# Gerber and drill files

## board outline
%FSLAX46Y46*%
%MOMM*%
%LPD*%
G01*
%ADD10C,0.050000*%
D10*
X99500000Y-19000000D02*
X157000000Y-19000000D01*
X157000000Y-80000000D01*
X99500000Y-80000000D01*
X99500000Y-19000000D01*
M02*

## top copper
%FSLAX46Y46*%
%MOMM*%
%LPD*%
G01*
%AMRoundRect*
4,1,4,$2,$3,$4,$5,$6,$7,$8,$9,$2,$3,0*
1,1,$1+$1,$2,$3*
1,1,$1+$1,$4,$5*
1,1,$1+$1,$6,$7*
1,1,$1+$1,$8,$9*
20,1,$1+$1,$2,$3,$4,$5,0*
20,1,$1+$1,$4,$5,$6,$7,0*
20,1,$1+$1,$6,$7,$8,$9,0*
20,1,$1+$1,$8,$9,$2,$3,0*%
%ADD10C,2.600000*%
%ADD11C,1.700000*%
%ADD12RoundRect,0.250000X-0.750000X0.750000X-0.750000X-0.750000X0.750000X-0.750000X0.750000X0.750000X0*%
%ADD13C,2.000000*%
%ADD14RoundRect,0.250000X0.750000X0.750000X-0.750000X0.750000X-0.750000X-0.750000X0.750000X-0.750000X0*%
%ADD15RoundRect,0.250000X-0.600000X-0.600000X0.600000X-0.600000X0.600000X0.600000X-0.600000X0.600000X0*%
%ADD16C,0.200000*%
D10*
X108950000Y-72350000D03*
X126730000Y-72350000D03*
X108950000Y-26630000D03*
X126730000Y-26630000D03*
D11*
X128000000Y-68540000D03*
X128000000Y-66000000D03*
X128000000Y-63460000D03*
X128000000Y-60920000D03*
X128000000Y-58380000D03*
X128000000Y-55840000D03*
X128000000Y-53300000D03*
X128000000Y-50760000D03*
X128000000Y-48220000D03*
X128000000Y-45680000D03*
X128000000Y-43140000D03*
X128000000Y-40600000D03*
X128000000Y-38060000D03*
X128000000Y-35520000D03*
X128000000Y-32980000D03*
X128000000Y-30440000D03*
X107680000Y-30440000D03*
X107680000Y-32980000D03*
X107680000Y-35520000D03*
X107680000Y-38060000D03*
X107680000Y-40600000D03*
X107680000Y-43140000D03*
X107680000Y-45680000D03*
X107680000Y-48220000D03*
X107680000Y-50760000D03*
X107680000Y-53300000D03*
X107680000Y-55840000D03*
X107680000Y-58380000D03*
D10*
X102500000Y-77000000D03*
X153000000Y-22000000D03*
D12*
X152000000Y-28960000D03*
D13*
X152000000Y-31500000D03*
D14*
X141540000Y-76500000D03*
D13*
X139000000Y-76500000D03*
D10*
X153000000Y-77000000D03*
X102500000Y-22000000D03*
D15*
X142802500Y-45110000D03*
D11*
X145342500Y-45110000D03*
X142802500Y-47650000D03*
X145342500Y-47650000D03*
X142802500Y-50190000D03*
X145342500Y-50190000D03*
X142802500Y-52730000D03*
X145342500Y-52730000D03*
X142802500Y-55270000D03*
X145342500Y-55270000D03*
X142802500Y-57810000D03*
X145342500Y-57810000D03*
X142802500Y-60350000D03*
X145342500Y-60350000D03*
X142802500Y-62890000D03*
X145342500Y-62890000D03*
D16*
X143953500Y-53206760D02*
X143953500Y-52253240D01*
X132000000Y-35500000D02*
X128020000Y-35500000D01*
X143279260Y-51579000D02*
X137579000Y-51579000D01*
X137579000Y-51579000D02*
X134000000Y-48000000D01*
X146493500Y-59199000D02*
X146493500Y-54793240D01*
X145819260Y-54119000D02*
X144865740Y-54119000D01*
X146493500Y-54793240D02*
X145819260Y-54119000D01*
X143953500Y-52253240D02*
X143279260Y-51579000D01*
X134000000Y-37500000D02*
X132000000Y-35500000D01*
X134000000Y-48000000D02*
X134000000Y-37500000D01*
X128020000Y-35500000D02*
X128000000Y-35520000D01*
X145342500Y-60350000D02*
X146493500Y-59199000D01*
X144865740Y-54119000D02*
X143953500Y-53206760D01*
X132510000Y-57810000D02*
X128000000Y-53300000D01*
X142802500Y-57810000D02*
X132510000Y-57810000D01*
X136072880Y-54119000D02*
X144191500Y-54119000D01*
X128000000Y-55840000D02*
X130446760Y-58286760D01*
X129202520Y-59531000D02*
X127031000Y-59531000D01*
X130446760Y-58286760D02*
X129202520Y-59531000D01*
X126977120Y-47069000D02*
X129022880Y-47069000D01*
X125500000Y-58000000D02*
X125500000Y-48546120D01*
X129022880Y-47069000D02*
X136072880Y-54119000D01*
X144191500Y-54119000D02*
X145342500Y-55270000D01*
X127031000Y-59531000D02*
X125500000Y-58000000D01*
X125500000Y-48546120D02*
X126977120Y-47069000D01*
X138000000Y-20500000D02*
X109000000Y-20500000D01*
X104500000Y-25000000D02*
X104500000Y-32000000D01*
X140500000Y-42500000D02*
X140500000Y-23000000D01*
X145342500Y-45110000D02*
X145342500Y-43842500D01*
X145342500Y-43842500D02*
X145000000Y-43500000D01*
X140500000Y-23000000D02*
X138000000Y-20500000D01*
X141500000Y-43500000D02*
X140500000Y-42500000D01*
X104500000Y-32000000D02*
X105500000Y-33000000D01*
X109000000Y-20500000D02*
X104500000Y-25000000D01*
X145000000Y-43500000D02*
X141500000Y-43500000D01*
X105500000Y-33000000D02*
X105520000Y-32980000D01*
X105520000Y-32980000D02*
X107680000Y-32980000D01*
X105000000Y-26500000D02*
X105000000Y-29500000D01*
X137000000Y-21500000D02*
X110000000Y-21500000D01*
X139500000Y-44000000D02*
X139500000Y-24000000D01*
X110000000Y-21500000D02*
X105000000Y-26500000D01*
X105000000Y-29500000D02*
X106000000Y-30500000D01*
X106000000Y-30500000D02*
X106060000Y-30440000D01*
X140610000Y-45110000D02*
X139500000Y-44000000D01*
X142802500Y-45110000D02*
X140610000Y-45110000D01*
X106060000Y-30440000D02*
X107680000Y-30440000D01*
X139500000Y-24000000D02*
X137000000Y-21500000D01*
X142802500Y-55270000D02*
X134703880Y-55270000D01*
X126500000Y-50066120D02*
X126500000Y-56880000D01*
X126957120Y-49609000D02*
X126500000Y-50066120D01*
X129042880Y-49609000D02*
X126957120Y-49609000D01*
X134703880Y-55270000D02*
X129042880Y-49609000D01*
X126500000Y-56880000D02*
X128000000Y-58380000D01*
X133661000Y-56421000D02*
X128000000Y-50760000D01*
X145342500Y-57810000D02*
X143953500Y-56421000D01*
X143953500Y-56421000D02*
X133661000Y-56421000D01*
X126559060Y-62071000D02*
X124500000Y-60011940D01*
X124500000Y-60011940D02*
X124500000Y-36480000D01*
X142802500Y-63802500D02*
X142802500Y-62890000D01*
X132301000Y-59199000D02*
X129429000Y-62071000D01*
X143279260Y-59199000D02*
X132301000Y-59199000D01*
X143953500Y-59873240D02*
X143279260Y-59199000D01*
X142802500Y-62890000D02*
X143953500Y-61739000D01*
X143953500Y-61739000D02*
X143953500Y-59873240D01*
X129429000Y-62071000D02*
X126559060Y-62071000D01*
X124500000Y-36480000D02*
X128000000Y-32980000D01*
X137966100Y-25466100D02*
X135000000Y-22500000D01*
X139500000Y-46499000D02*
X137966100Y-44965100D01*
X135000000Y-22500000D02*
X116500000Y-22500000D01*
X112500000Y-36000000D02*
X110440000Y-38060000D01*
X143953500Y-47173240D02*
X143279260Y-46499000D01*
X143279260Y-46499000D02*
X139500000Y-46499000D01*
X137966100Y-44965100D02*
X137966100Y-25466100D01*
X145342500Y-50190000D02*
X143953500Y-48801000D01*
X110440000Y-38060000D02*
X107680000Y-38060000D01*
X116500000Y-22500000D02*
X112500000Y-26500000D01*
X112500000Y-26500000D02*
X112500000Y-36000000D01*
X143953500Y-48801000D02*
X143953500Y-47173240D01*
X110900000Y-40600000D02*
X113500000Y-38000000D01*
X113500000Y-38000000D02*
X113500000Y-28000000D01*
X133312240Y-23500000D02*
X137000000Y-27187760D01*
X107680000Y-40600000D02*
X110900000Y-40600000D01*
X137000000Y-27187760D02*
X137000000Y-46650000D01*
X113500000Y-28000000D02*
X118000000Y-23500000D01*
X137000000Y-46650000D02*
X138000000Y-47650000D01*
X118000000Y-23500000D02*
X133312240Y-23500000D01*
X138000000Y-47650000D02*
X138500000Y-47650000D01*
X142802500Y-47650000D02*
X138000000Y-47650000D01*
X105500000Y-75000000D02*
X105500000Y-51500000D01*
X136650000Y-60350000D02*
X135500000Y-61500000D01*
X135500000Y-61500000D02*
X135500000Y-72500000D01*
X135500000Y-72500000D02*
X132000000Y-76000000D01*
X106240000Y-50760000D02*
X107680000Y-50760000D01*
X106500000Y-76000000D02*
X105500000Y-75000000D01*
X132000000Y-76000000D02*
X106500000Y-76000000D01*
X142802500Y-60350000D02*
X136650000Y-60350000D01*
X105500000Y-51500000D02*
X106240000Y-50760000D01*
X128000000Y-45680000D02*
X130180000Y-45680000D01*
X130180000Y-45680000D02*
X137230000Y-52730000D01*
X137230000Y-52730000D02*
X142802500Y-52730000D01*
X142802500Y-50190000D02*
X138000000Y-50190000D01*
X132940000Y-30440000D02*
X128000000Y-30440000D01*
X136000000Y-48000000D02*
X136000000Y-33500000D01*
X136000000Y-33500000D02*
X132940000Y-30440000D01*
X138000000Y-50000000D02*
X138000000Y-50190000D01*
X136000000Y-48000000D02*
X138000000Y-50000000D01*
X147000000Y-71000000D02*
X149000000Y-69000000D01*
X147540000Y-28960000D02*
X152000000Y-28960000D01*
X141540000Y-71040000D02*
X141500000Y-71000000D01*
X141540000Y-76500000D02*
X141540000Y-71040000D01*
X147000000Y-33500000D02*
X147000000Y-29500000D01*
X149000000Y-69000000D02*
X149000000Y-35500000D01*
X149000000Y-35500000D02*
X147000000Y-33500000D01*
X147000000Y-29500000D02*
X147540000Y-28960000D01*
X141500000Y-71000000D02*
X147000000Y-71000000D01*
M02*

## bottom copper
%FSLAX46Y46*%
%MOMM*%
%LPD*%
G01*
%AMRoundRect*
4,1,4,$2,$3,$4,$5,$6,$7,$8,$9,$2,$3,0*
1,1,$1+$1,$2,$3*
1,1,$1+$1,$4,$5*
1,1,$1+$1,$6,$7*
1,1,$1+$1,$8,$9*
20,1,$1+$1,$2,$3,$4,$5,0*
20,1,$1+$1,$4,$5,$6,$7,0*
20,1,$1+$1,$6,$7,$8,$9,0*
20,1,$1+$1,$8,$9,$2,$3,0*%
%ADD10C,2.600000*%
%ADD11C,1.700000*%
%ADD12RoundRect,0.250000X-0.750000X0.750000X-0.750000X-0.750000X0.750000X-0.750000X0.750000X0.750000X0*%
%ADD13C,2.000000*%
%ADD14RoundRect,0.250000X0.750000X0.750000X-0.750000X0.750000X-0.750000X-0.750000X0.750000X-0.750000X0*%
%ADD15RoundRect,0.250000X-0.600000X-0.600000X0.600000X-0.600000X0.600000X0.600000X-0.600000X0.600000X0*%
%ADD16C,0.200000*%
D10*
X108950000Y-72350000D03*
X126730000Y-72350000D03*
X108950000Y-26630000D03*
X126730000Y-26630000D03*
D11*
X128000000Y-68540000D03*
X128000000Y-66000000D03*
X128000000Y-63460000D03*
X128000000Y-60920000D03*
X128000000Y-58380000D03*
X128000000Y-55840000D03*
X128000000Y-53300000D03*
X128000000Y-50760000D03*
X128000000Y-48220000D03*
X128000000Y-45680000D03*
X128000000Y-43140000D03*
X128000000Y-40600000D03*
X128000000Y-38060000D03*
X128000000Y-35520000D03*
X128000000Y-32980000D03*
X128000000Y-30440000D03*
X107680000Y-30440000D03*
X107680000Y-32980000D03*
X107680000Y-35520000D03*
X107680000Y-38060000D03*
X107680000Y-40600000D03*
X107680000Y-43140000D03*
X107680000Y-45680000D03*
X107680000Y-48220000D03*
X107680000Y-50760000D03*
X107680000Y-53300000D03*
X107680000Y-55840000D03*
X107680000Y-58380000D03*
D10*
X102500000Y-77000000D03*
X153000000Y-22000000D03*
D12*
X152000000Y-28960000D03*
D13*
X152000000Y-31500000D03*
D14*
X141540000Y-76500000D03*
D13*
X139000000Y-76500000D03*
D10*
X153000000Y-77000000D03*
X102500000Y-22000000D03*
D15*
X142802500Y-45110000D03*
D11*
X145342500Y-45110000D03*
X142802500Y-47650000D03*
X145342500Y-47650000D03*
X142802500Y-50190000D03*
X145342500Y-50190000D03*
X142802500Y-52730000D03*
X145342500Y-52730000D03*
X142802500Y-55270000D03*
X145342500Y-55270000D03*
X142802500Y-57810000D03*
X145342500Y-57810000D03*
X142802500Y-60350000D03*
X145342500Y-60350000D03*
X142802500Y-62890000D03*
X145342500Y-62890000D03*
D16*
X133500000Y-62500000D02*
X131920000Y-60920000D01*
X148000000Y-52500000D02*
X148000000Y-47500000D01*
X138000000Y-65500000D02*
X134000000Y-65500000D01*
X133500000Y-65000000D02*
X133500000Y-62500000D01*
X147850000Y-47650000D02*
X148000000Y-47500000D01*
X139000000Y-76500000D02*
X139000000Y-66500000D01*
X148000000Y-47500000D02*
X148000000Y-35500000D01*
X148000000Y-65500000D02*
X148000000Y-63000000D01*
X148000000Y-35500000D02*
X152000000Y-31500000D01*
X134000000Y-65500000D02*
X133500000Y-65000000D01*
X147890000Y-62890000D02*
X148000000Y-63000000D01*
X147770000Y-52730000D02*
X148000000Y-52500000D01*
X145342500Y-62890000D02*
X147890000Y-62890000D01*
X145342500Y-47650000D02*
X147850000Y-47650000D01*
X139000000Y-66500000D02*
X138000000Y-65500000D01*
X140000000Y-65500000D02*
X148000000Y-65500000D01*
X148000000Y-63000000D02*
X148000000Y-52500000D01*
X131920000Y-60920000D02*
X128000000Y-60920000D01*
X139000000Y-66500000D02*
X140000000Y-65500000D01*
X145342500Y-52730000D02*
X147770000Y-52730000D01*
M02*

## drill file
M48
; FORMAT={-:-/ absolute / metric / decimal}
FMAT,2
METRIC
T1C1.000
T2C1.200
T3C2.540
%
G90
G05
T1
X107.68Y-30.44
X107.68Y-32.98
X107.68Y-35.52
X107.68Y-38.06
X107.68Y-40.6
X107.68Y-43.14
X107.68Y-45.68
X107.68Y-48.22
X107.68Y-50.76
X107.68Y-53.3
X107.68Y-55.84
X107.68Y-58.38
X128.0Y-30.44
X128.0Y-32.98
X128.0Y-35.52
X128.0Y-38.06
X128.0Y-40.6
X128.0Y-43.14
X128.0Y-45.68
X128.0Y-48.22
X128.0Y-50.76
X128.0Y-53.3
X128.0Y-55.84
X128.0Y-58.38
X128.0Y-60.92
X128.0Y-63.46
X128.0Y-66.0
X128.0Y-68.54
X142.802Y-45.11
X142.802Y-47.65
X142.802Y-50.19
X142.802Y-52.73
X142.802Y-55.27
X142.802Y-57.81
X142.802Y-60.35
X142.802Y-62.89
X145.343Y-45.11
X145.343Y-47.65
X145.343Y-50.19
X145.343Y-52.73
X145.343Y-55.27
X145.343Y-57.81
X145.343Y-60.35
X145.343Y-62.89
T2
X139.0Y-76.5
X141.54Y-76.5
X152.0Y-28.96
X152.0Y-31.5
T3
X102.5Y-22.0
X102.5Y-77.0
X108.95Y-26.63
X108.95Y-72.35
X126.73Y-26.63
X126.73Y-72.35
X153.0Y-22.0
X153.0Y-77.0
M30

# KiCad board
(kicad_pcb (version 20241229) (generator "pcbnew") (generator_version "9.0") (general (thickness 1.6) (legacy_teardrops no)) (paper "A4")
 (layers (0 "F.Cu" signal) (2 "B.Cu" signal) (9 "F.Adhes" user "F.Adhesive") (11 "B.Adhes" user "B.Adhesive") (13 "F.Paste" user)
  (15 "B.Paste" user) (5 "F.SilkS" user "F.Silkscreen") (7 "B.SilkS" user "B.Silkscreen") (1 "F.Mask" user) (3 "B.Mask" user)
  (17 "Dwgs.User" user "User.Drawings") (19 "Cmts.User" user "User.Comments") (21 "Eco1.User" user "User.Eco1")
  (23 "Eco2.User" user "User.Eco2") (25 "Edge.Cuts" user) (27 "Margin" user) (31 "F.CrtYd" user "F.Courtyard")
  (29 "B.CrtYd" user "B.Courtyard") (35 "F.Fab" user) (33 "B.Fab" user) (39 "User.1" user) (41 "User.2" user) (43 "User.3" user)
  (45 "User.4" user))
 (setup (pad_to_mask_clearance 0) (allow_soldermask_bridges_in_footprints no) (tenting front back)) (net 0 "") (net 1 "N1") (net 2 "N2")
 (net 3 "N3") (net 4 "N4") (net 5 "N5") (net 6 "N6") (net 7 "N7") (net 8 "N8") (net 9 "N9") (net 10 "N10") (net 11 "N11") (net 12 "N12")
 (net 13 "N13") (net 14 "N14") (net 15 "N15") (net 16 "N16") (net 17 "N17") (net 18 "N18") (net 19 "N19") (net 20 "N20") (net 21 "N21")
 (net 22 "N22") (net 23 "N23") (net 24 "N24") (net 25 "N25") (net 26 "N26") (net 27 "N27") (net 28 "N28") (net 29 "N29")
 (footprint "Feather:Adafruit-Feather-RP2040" (layer "F.Cu") (at 117.84 49.49 90)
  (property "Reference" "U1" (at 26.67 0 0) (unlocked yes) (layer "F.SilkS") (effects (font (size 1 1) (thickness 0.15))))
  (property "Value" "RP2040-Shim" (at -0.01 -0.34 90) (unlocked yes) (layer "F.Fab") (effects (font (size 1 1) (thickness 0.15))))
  (pad "" np_thru_hole circle (at -22.86 -8.89 90) (size 2.6 2.6) (drill 2.54) (layers "*.Cu" "*.Mask") (solder_mask_margin 1.3)
   (clearance 1.3))
  (pad "" np_thru_hole circle (at -22.86 8.89 90) (size 2.6 2.6) (drill 2.54) (layers "*.Cu" "*.Mask") (solder_mask_margin 1.3)
   (clearance 1.3))
  (pad "" np_thru_hole circle (at 22.86 -8.89 90) (size 2.6 2.6) (drill 2.54) (layers "*.Cu" "*.Mask") (solder_mask_margin 1.3)
   (clearance 1.3))
  (pad "" np_thru_hole circle (at 22.86 8.89 90) (size 2.6 2.6) (drill 2.54) (layers "*.Cu" "*.Mask") (solder_mask_margin 1.3)
   (clearance 1.3))
  (pad "1" thru_hole circle (at -19.05 10.16 90) (size 1.7 1.7) (drill 1) (layers "*.Cu" "*.Mask") (remove_unused_layers no) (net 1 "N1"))
  (pad "2" thru_hole circle (at -16.51 10.16 90) (size 1.7 1.7) (drill 1) (layers "*.Cu" "*.Mask") (remove_unused_layers no) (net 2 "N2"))
  (pad "3" thru_hole circle (at -13.97 10.16 90) (size 1.7 1.7) (drill 1) (layers "*.Cu" "*.Mask") (remove_unused_layers no) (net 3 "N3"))
  (pad "4" thru_hole circle (at -11.43 10.16 90) (size 1.7 1.7) (drill 1) (layers "*.Cu" "*.Mask") (remove_unused_layers no) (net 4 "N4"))
  (pad "5" thru_hole circle (at -8.89 10.16 90) (size 1.7 1.7) (drill 1) (layers "*.Cu" "*.Mask") (remove_unused_layers no) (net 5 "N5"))
  (pad "6" thru_hole circle (at -6.35 10.16 90) (size 1.7 1.7) (drill 1) (layers "*.Cu" "*.Mask") (remove_unused_layers no) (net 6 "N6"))
  (pad "7" thru_hole circle (at -3.81 10.16 90) (size 1.7 1.7) (drill 1) (layers "*.Cu" "*.Mask") (remove_unused_layers no) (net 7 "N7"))
  (pad "8" thru_hole circle (at -1.27 10.16 90) (size 1.7 1.7) (drill 1) (layers "*.Cu" "*.Mask") (remove_unused_layers no) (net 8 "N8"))
  (pad "9" thru_hole circle (at 1.27 10.16 90) (size 1.7 1.7) (drill 1) (layers "*.Cu" "*.Mask") (remove_unused_layers no) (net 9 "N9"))
  (pad "10" thru_hole circle (at 3.81 10.16 90) (size 1.7 1.7) (drill 1) (layers "*.Cu" "*.Mask") (remove_unused_layers no) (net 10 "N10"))
  (pad "11" thru_hole circle (at 6.35 10.16 90) (size 1.7 1.7) (drill 1) (layers "*.Cu" "*.Mask") (remove_unused_layers no) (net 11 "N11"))
  (pad "12" thru_hole circle (at 8.89 10.16 90) (size 1.7 1.7) (drill 1) (layers "*.Cu" "*.Mask") (remove_unused_layers no) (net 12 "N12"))
  (pad "13" thru_hole circle (at 11.43 10.16 90) (size 1.7 1.7) (drill 1) (layers "*.Cu" "*.Mask") (remove_unused_layers no) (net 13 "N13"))
  (pad "14" thru_hole circle (at 13.97 10.16 90) (size 1.7 1.7) (drill 1) (layers "*.Cu" "*.Mask") (remove_unused_layers no) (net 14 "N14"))
  (pad "15" thru_hole circle (at 16.51 10.16 90) (size 1.7 1.7) (drill 1) (layers "*.Cu" "*.Mask") (remove_unused_layers no) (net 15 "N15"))
  (pad "16" thru_hole circle (at 19.05 10.16 90) (size 1.7 1.7) (drill 1) (layers "*.Cu" "*.Mask") (remove_unused_layers no) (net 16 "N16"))
  (pad "17" thru_hole circle (at 19.05 -10.16 90) (size 1.7 1.7) (drill 1) (layers "*.Cu" "*.Mask") (remove_unused_layers no) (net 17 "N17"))
  (pad "18" thru_hole circle (at 16.51 -10.16 90) (size 1.7 1.7) (drill 1) (layers "*.Cu" "*.Mask") (remove_unused_layers no) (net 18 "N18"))
  (pad "19" thru_hole circle (at 13.97 -10.16 90) (size 1.7 1.7) (drill 1) (layers "*.Cu" "*.Mask") (remove_unused_layers no) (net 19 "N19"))
  (pad "20" thru_hole circle (at 11.43 -10.16 90) (size 1.7 1.7) (drill 1) (layers "*.Cu" "*.Mask") (remove_unused_layers no) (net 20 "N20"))
  (pad "21" thru_hole circle (at 8.89 -10.16 90) (size 1.7 1.7) (drill 1) (layers "*.Cu" "*.Mask") (remove_unused_layers no) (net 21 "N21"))
  (pad "22" thru_hole circle (at 6.35 -10.16 90) (size 1.7 1.7) (drill 1) (layers "*.Cu" "*.Mask") (remove_unused_layers no) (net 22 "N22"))
  (pad "23" thru_hole circle (at 3.81 -10.16 90) (size 1.7 1.7) (drill 1) (layers "*.Cu" "*.Mask") (remove_unused_layers no) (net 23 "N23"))
  (pad "24" thru_hole circle (at 1.27 -10.16 90) (size 1.7 1.7) (drill 1) (layers "*.Cu" "*.Mask") (remove_unused_layers no) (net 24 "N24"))
  (pad "25" thru_hole circle (at -1.27 -10.16 90) (size 1.7 1.7) (drill 1) (layers "*.Cu" "*.Mask") (remove_unused_layers no) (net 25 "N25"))
  (pad "26" thru_hole circle (at -3.81 -10.16 90) (size 1.7 1.7) (drill 1) (layers "*.Cu" "*.Mask") (remove_unused_layers no) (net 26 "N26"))
  (pad "27" thru_hole circle (at -6.35 -10.16 90) (size 1.7 1.7) (drill 1) (layers "*.Cu" "*.Mask") (remove_unused_layers no) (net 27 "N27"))
  (pad "28" thru_hole circle (at -8.89 -10.16 90) (size 1.7 1.7) (drill 1) (layers "*.Cu" "*.Mask") (remove_unused_layers no) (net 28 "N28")))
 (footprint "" (layer "F.Cu") (at 102.5 77)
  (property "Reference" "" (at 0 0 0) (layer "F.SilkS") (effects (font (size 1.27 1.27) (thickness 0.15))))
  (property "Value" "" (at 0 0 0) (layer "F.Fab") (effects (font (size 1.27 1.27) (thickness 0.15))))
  (pad "" np_thru_hole circle (at 0 0 90) (size 2.6 2.6) (drill 2.54) (layers "*.Cu" "*.Mask") (solder_mask_margin 1.3) (clearance 1.3)))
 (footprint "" (layer "F.Cu") (at 153 22)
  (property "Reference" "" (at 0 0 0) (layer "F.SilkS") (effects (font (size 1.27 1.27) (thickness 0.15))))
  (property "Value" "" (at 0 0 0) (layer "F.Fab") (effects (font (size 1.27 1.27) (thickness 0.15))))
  (pad "" np_thru_hole circle (at 0 0 90) (size 2.6 2.6) (drill 2.54) (layers "*.Cu" "*.Mask") (solder_mask_margin 1.3) (clearance 1.3)))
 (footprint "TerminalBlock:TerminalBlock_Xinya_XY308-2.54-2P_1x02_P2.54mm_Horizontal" (layer "F.Cu") (at 152 28.96 -90)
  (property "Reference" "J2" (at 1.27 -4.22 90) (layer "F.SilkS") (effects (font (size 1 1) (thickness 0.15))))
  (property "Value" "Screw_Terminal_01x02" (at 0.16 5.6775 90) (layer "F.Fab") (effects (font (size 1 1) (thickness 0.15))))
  (pad "1" thru_hole roundrect (at 0 0 270) (size 2 2) (drill 1.2) (layers "*.Cu" "*.Mask") (remove_unused_layers no)
   (roundrect_rratio 0.125) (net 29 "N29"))
  (pad "2" thru_hole circle (at 2.54 0 270) (size 2 2) (drill 1.2) (layers "*.Cu" "*.Mask") (remove_unused_layers no) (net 4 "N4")))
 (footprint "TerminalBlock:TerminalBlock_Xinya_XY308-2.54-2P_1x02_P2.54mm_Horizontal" (layer "F.Cu") (at 141.54 76.5 180)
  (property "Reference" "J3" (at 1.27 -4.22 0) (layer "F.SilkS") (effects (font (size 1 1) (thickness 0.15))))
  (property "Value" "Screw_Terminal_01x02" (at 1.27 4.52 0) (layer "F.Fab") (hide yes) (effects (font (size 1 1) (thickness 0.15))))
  (pad "1" thru_hole roundrect (at 0 0 180) (size 2 2) (drill 1.2) (layers "*.Cu" "*.Mask") (remove_unused_layers no)
   (roundrect_rratio 0.125) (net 29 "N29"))
  (pad "2" thru_hole circle (at 2.54 0 180) (size 2 2) (drill 1.2) (layers "*.Cu" "*.Mask") (remove_unused_layers no) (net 4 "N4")))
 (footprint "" (layer "F.Cu") (at 153 77)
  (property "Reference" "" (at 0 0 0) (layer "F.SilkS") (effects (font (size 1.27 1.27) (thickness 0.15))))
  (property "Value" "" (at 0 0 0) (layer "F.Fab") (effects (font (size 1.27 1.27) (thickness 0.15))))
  (pad "" np_thru_hole circle (at 0 0 90) (size 2.6 2.6) (drill 2.54) (layers "*.Cu" "*.Mask") (solder_mask_margin 1.3) (clearance 1.3)))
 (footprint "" (layer "F.Cu") (at 102.5 22)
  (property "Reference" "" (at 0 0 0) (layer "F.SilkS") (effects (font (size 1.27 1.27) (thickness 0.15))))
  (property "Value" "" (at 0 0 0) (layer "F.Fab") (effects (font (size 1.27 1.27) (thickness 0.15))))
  (pad "" np_thru_hole circle (at 0 0 90) (size 2.6 2.6) (drill 2.54) (layers "*.Cu" "*.Mask") (solder_mask_margin 1.3) (clearance 1.3)))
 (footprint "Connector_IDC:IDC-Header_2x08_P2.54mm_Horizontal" (layer "F.Cu") (at 142.8025 45.11)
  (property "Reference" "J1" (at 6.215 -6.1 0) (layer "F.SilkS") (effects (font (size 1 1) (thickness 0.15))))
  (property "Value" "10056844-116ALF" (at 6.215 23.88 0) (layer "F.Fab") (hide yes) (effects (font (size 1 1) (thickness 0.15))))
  (pad "1" thru_hole roundrect (at 0 0) (size 1.7 1.7) (drill 1) (layers "*.Cu" "*.Mask") (remove_unused_layers no)
   (roundrect_rratio 0.147059) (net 17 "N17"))
  (pad "2" thru_hole circle (at 2.54 0) (size 1.7 1.7) (drill 1) (layers "*.Cu" "*.Mask") (remove_unused_layers no) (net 18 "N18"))
  (pad "3" thru_hole circle (at 0 2.54) (size 1.7 1.7) (drill 1) (layers "*.Cu" "*.Mask") (remove_unused_layers no) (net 21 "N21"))
  (pad "4" thru_hole circle (at 2.54 2.54) (size 1.7 1.7) (drill 1) (layers "*.Cu" "*.Mask") (remove_unused_layers no) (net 4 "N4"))
  (pad "5" thru_hole circle (at 0 5.08) (size 1.7 1.7) (drill 1) (layers "*.Cu" "*.Mask") (remove_unused_layers no) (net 16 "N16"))
  (pad "6" thru_hole circle (at 2.54 5.08) (size 1.7 1.7) (drill 1) (layers "*.Cu" "*.Mask") (remove_unused_layers no) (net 20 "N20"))
  (pad "7" thru_hole circle (at 0 7.62) (size 1.7 1.7) (drill 1) (layers "*.Cu" "*.Mask") (remove_unused_layers no) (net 10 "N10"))
  (pad "8" thru_hole circle (at 2.54 7.62) (size 1.7 1.7) (drill 1) (layers "*.Cu" "*.Mask") (remove_unused_layers no) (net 4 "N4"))
  (pad "9" thru_hole circle (at 0 10.16) (size 1.7 1.7) (drill 1) (layers "*.Cu" "*.Mask") (remove_unused_layers no) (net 5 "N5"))
  (pad "10" thru_hole circle (at 2.54 10.16) (size 1.7 1.7) (drill 1) (layers "*.Cu" "*.Mask") (remove_unused_layers no) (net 6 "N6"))
  (pad "11" thru_hole circle (at 0 12.7) (size 1.7 1.7) (drill 1) (layers "*.Cu" "*.Mask") (remove_unused_layers no) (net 7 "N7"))
  (pad "12" thru_hole circle (at 2.54 12.7) (size 1.7 1.7) (drill 1) (layers "*.Cu" "*.Mask") (remove_unused_layers no) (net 8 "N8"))
  (pad "13" thru_hole circle (at 0 15.24) (size 1.7 1.7) (drill 1) (layers "*.Cu" "*.Mask") (remove_unused_layers no) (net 25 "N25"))
  (pad "14" thru_hole circle (at 2.54 15.24) (size 1.7 1.7) (drill 1) (layers "*.Cu" "*.Mask") (remove_unused_layers no) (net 14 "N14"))
  (pad "15" thru_hole circle (at 0 17.78) (size 1.7 1.7) (drill 1) (layers "*.Cu" "*.Mask") (remove_unused_layers no) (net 15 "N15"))
  (pad "16" thru_hole circle (at 2.54 17.78) (size 1.7 1.7) (drill 1) (layers "*.Cu" "*.Mask") (remove_unused_layers no) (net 4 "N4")))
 (gr_rect (start 99.5 19) (end 157 80) (stroke (width 0.05) (type solid)) (fill no) (layer "Edge.Cuts"))
 (segment (start 143.9535 53.20676) (end 143.9535 52.25324) (width 0.2) (layer "F.Cu") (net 14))
 (segment (start 132 35.5) (end 128.02 35.5) (width 0.2) (layer "F.Cu") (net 14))
 (segment (start 143.27926 51.579) (end 137.579 51.579) (width 0.2) (layer "F.Cu") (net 14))
 (segment (start 137.579 51.579) (end 134 48) (width 0.2) (layer "F.Cu") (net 14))
 (segment (start 146.4935 59.199) (end 146.4935 54.79324) (width 0.2) (layer "F.Cu") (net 14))
 (segment (start 145.81926 54.119) (end 144.86574 54.119) (width 0.2) (layer "F.Cu") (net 14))
 (segment (start 146.4935 54.79324) (end 145.81926 54.119) (width 0.2) (layer "F.Cu") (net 14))
 (segment (start 143.9535 52.25324) (end 143.27926 51.579) (width 0.2) (layer "F.Cu") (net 14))
 (segment (start 134 37.5) (end 132 35.5) (width 0.2) (layer "F.Cu") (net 14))
 (segment (start 134 48) (end 134 37.5) (width 0.2) (layer "F.Cu") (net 14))
 (segment (start 128.02 35.5) (end 128 35.52) (width 0.2) (layer "F.Cu") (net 14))
 (segment (start 145.3425 60.35) (end 146.4935 59.199) (width 0.2) (layer "F.Cu") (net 14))
 (segment (start 144.86574 54.119) (end 143.9535 53.20676) (width 0.2) (layer "F.Cu") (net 14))
 (segment (start 132.51 57.81) (end 128 53.3) (width 0.2) (layer "F.Cu") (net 7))
 (segment (start 142.8025 57.81) (end 132.51 57.81) (width 0.2) (layer "F.Cu") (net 7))
 (segment (start 136.07288 54.119) (end 144.1915 54.119) (width 0.2) (layer "F.Cu") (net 6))
 (segment (start 128 55.84) (end 130.44676 58.28676) (width 0.2) (layer "F.Cu") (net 6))
 (segment (start 129.20252 59.531) (end 127.031 59.531) (width 0.2) (layer "F.Cu") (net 6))
 (segment (start 130.44676 58.28676) (end 129.20252 59.531) (width 0.2) (layer "F.Cu") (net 6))
 (segment (start 126.97712 47.069) (end 129.02288 47.069) (width 0.2) (layer "F.Cu") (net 6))
 (segment (start 125.5 58) (end 125.5 48.54612) (width 0.2) (layer "F.Cu") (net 6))
 (segment (start 129.02288 47.069) (end 136.07288 54.119) (width 0.2) (layer "F.Cu") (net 6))
 (segment (start 144.1915 54.119) (end 145.3425 55.27) (width 0.2) (layer "F.Cu") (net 6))
 (segment (start 127.031 59.531) (end 125.5 58) (width 0.2) (layer "F.Cu") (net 6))
 (segment (start 125.5 48.54612) (end 126.97712 47.069) (width 0.2) (layer "F.Cu") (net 6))
 (segment (start 138 20.5) (end 109 20.5) (width 0.2) (layer "F.Cu") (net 18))
 (segment (start 104.5 25) (end 104.5 32) (width 0.2) (layer "F.Cu") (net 18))
 (segment (start 140.5 42.5) (end 140.5 23) (width 0.2) (layer "F.Cu") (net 18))
 (segment (start 145.3425 45.11) (end 145.3425 43.8425) (width 0.2) (layer "F.Cu") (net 18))
 (segment (start 145.3425 43.8425) (end 145 43.5) (width 0.2) (layer "F.Cu") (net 18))
 (segment (start 140.5 23) (end 138 20.5) (width 0.2) (layer "F.Cu") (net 18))
 (segment (start 141.5 43.5) (end 140.5 42.5) (width 0.2) (layer "F.Cu") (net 18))
 (segment (start 104.5 32) (end 105.5 33) (width 0.2) (layer "F.Cu") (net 18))
 (segment (start 109 20.5) (end 104.5 25) (width 0.2) (layer "F.Cu") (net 18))
 (segment (start 145 43.5) (end 141.5 43.5) (width 0.2) (layer "F.Cu") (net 18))
 (segment (start 105.5 33) (end 105.52 32.98) (width 0.2) (layer "F.Cu") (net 18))
 (segment (start 105.52 32.98) (end 107.68 32.98) (width 0.2) (layer "F.Cu") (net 18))
 (segment (start 105 26.5) (end 105 29.5) (width 0.2) (layer "F.Cu") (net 17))
 (segment (start 137 21.5) (end 110 21.5) (width 0.2) (layer "F.Cu") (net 17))
 (segment (start 139.5 44) (end 139.5 24) (width 0.2) (layer "F.Cu") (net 17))
 (segment (start 110 21.5) (end 105 26.5) (width 0.2) (layer "F.Cu") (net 17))
 (segment (start 105 29.5) (end 106 30.5) (width 0.2) (layer "F.Cu") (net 17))
 (segment (start 106 30.5) (end 106.06 30.44) (width 0.2) (layer "F.Cu") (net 17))
 (segment (start 140.61 45.11) (end 139.5 44) (width 0.2) (layer "F.Cu") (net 17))
 (segment (start 142.8025 45.11) (end 140.61 45.11) (width 0.2) (layer "F.Cu") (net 17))
 (segment (start 106.06 30.44) (end 107.68 30.44) (width 0.2) (layer "F.Cu") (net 17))
 (segment (start 139.5 24) (end 137 21.5) (width 0.2) (layer "F.Cu") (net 17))
 (segment (start 142.8025 55.27) (end 134.70388 55.27) (width 0.2) (layer "F.Cu") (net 5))
 (segment (start 126.5 50.06612) (end 126.5 56.88) (width 0.2) (layer "F.Cu") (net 5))
 (segment (start 126.95712 49.609) (end 126.5 50.06612) (width 0.2) (layer "F.Cu") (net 5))
 (segment (start 129.04288 49.609) (end 126.95712 49.609) (width 0.2) (layer "F.Cu") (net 5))
 (segment (start 134.70388 55.27) (end 129.04288 49.609) (width 0.2) (layer "F.Cu") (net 5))
 (segment (start 126.5 56.88) (end 128 58.38) (width 0.2) (layer "F.Cu") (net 5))
 (segment (start 133.661 56.421) (end 128 50.76) (width 0.2) (layer "F.Cu") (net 8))
 (segment (start 145.3425 57.81) (end 143.9535 56.421) (width 0.2) (layer "F.Cu") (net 8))
 (segment (start 143.9535 56.421) (end 133.661 56.421) (width 0.2) (layer "F.Cu") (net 8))
 (segment (start 133.5 62.5) (end 131.92 60.92) (width 0.2) (layer "B.Cu") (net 4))
 (segment (start 148 52.5) (end 148 47.5) (width 0.2) (layer "B.Cu") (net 4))
 (segment (start 138 65.5) (end 134 65.5) (width 0.2) (layer "B.Cu") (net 4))
 (segment (start 133.5 65) (end 133.5 62.5) (width 0.2) (layer "B.Cu") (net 4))
 (segment (start 147.85 47.65) (end 148 47.5) (width 0.2) (layer "B.Cu") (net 4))
 (segment (start 139 76.5) (end 139 66.5) (width 0.2) (layer "B.Cu") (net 4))
 (segment (start 148 47.5) (end 148 35.5) (width 0.2) (layer "B.Cu") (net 4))
 (segment (start 148 65.5) (end 148 63) (width 0.2) (layer "B.Cu") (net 4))
 (segment (start 148 35.5) (end 152 31.5) (width 0.2) (layer "B.Cu") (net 4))
 (segment (start 134 65.5) (end 133.5 65) (width 0.2) (layer "B.Cu") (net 4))
 (segment (start 147.89 62.89) (end 148 63) (width 0.2) (layer "B.Cu") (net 4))
 (segment (start 147.77 52.73) (end 148 52.5) (width 0.2) (layer "B.Cu") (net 4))
 (segment (start 145.3425 62.89) (end 147.89 62.89) (width 0.2) (layer "B.Cu") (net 4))
 (segment (start 145.3425 47.65) (end 147.85 47.65) (width 0.2) (layer "B.Cu") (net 4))
 (segment (start 139 66.5) (end 138 65.5) (width 0.2) (layer "B.Cu") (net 4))
 (segment (start 140 65.5) (end 148 65.5) (width 0.2) (layer "B.Cu") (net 4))
 (segment (start 148 63) (end 148 52.5) (width 0.2) (layer "B.Cu") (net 4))
 (segment (start 131.92 60.92) (end 128 60.92) (width 0.2) (layer "B.Cu") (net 4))
 (segment (start 139 66.5) (end 140 65.5) (width 0.2) (layer "B.Cu") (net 4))
 (segment (start 145.3425 52.73) (end 147.77 52.73) (width 0.2) (layer "B.Cu") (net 4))
 (segment (start 126.55906 62.071) (end 124.5 60.01194) (width 0.2) (layer "F.Cu") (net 15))
 (segment (start 124.5 60.01194) (end 124.5 36.48) (width 0.2) (layer "F.Cu") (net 15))
 (segment (start 142.8025 63.8025) (end 142.8025 62.89) (width 0.2) (layer "F.Cu") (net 15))
 (segment (start 132.301 59.199) (end 129.429 62.071) (width 0.2) (layer "F.Cu") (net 15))
 (segment (start 143.27926 59.199) (end 132.301 59.199) (width 0.2) (layer "F.Cu") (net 15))
 (segment (start 143.9535 59.87324) (end 143.27926 59.199) (width 0.2) (layer "F.Cu") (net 15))
 (segment (start 142.8025 62.89) (end 143.9535 61.739) (width 0.2) (layer "F.Cu") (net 15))
 (segment (start 143.9535 61.739) (end 143.9535 59.87324) (width 0.2) (layer "F.Cu") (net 15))
 (segment (start 129.429 62.071) (end 126.55906 62.071) (width 0.2) (layer "F.Cu") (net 15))
 (segment (start 124.5 36.48) (end 128 32.98) (width 0.2) (layer "F.Cu") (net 15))
 (segment (start 137.9661 25.4661) (end 135 22.5) (width 0.2) (layer "F.Cu") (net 20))
 (segment (start 139.5 46.499) (end 137.9661 44.9651) (width 0.2) (layer "F.Cu") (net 20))
 (segment (start 135 22.5) (end 116.5 22.5) (width 0.2) (layer "F.Cu") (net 20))
 (segment (start 112.5 36) (end 110.44 38.06) (width 0.2) (layer "F.Cu") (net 20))
 (segment (start 143.9535 47.17324) (end 143.27926 46.499) (width 0.2) (layer "F.Cu") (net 20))
 (segment (start 143.27926 46.499) (end 139.5 46.499) (width 0.2) (layer "F.Cu") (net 20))
 (segment (start 137.9661 44.9651) (end 137.9661 25.4661) (width 0.2) (layer "F.Cu") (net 20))
 (segment (start 145.3425 50.19) (end 143.9535 48.801) (width 0.2) (layer "F.Cu") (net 20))
 (segment (start 110.44 38.06) (end 107.68 38.06) (width 0.2) (layer "F.Cu") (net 20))
 (segment (start 116.5 22.5) (end 112.5 26.5) (width 0.2) (layer "F.Cu") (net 20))
 (segment (start 112.5 26.5) (end 112.5 36) (width 0.2) (layer "F.Cu") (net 20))
 (segment (start 143.9535 48.801) (end 143.9535 47.17324) (width 0.2) (layer "F.Cu") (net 20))
 (segment (start 110.9 40.6) (end 113.5 38) (width 0.2) (layer "F.Cu") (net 21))
 (segment (start 113.5 38) (end 113.5 28) (width 0.2) (layer "F.Cu") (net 21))
 (segment (start 133.31224 23.5) (end 137 27.18776) (width 0.2) (layer "F.Cu") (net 21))
 (segment (start 107.68 40.6) (end 110.9 40.6) (width 0.2) (layer "F.Cu") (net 21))
 (segment (start 137 27.18776) (end 137 46.65) (width 0.2) (layer "F.Cu") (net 21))
 (segment (start 113.5 28) (end 118 23.5) (width 0.2) (layer "F.Cu") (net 21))
 (segment (start 137 46.65) (end 138 47.65) (width 0.2) (layer "F.Cu") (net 21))
 (segment (start 118 23.5) (end 133.31224 23.5) (width 0.2) (layer "F.Cu") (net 21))
 (segment (start 138 47.65) (end 138.5 47.65) (width 0.2) (layer "F.Cu") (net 21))
 (segment (start 142.8025 47.65) (end 138 47.65) (width 0.2) (layer "F.Cu") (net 21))
 (segment (start 105.5 75) (end 105.5 51.5) (width 0.2) (layer "F.Cu") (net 25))
 (segment (start 136.65 60.35) (end 135.5 61.5) (width 0.2) (layer "F.Cu") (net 25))
 (segment (start 135.5 61.5) (end 135.5 72.5) (width 0.2) (layer "F.Cu") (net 25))
 (segment (start 135.5 72.5) (end 132 76) (width 0.2) (layer "F.Cu") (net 25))
 (segment (start 106.24 50.76) (end 107.68 50.76) (width 0.2) (layer "F.Cu") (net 25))
 (segment (start 106.5 76) (end 105.5 75) (width 0.2) (layer "F.Cu") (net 25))
 (segment (start 132 76) (end 106.5 76) (width 0.2) (layer "F.Cu") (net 25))
 (segment (start 142.8025 60.35) (end 136.65 60.35) (width 0.2) (layer "F.Cu") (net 25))
 (segment (start 105.5 51.5) (end 106.24 50.76) (width 0.2) (layer "F.Cu") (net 25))
 (segment (start 128 45.68) (end 130.18 45.68) (width 0.2) (layer "F.Cu") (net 10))
 (segment (start 130.18 45.68) (end 137.23 52.73) (width 0.2) (layer "F.Cu") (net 10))
 (segment (start 137.23 52.73) (end 142.8025 52.73) (width 0.2) (layer "F.Cu") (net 10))
 (segment (start 142.8025 50.19) (end 138 50.19) (width 0.2) (layer "F.Cu") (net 16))
 (segment (start 132.94 30.44) (end 128 30.44) (width 0.2) (layer "F.Cu") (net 16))
 (segment (start 136 48) (end 136 33.5) (width 0.2) (layer "F.Cu") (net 16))
 (segment (start 136 33.5) (end 132.94 30.44) (width 0.2) (layer "F.Cu") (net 16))
 (segment (start 138 50) (end 138 50.19) (width 0.2) (layer "F.Cu") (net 16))
 (segment (start 136 48) (end 138 50) (width 0.2) (layer "F.Cu") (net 16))
 (segment (start 147 71) (end 149 69) (width 0.2) (layer "F.Cu") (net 29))
 (segment (start 147.54 28.96) (end 152 28.96) (width 0.2) (layer "F.Cu") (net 29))
 (segment (start 141.54 71.04) (end 141.5 71) (width 0.2) (layer "F.Cu") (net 29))
 (segment (start 141.54 76.5) (end 141.54 71.04) (width 0.2) (layer "F.Cu") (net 29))
 (segment (start 147 33.5) (end 147 29.5) (width 0.2) (layer "F.Cu") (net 29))
 (segment (start 149 69) (end 149 35.5) (width 0.2) (layer "F.Cu") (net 29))
 (segment (start 149 35.5) (end 147 33.5) (width 0.2) (layer "F.Cu") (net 29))
 (segment (start 147 29.5) (end 147.54 28.96) (width 0.2) (layer "F.Cu") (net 29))
 (segment (start 141.5 71) (end 147 71) (width 0.2) (layer "F.Cu") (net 29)))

